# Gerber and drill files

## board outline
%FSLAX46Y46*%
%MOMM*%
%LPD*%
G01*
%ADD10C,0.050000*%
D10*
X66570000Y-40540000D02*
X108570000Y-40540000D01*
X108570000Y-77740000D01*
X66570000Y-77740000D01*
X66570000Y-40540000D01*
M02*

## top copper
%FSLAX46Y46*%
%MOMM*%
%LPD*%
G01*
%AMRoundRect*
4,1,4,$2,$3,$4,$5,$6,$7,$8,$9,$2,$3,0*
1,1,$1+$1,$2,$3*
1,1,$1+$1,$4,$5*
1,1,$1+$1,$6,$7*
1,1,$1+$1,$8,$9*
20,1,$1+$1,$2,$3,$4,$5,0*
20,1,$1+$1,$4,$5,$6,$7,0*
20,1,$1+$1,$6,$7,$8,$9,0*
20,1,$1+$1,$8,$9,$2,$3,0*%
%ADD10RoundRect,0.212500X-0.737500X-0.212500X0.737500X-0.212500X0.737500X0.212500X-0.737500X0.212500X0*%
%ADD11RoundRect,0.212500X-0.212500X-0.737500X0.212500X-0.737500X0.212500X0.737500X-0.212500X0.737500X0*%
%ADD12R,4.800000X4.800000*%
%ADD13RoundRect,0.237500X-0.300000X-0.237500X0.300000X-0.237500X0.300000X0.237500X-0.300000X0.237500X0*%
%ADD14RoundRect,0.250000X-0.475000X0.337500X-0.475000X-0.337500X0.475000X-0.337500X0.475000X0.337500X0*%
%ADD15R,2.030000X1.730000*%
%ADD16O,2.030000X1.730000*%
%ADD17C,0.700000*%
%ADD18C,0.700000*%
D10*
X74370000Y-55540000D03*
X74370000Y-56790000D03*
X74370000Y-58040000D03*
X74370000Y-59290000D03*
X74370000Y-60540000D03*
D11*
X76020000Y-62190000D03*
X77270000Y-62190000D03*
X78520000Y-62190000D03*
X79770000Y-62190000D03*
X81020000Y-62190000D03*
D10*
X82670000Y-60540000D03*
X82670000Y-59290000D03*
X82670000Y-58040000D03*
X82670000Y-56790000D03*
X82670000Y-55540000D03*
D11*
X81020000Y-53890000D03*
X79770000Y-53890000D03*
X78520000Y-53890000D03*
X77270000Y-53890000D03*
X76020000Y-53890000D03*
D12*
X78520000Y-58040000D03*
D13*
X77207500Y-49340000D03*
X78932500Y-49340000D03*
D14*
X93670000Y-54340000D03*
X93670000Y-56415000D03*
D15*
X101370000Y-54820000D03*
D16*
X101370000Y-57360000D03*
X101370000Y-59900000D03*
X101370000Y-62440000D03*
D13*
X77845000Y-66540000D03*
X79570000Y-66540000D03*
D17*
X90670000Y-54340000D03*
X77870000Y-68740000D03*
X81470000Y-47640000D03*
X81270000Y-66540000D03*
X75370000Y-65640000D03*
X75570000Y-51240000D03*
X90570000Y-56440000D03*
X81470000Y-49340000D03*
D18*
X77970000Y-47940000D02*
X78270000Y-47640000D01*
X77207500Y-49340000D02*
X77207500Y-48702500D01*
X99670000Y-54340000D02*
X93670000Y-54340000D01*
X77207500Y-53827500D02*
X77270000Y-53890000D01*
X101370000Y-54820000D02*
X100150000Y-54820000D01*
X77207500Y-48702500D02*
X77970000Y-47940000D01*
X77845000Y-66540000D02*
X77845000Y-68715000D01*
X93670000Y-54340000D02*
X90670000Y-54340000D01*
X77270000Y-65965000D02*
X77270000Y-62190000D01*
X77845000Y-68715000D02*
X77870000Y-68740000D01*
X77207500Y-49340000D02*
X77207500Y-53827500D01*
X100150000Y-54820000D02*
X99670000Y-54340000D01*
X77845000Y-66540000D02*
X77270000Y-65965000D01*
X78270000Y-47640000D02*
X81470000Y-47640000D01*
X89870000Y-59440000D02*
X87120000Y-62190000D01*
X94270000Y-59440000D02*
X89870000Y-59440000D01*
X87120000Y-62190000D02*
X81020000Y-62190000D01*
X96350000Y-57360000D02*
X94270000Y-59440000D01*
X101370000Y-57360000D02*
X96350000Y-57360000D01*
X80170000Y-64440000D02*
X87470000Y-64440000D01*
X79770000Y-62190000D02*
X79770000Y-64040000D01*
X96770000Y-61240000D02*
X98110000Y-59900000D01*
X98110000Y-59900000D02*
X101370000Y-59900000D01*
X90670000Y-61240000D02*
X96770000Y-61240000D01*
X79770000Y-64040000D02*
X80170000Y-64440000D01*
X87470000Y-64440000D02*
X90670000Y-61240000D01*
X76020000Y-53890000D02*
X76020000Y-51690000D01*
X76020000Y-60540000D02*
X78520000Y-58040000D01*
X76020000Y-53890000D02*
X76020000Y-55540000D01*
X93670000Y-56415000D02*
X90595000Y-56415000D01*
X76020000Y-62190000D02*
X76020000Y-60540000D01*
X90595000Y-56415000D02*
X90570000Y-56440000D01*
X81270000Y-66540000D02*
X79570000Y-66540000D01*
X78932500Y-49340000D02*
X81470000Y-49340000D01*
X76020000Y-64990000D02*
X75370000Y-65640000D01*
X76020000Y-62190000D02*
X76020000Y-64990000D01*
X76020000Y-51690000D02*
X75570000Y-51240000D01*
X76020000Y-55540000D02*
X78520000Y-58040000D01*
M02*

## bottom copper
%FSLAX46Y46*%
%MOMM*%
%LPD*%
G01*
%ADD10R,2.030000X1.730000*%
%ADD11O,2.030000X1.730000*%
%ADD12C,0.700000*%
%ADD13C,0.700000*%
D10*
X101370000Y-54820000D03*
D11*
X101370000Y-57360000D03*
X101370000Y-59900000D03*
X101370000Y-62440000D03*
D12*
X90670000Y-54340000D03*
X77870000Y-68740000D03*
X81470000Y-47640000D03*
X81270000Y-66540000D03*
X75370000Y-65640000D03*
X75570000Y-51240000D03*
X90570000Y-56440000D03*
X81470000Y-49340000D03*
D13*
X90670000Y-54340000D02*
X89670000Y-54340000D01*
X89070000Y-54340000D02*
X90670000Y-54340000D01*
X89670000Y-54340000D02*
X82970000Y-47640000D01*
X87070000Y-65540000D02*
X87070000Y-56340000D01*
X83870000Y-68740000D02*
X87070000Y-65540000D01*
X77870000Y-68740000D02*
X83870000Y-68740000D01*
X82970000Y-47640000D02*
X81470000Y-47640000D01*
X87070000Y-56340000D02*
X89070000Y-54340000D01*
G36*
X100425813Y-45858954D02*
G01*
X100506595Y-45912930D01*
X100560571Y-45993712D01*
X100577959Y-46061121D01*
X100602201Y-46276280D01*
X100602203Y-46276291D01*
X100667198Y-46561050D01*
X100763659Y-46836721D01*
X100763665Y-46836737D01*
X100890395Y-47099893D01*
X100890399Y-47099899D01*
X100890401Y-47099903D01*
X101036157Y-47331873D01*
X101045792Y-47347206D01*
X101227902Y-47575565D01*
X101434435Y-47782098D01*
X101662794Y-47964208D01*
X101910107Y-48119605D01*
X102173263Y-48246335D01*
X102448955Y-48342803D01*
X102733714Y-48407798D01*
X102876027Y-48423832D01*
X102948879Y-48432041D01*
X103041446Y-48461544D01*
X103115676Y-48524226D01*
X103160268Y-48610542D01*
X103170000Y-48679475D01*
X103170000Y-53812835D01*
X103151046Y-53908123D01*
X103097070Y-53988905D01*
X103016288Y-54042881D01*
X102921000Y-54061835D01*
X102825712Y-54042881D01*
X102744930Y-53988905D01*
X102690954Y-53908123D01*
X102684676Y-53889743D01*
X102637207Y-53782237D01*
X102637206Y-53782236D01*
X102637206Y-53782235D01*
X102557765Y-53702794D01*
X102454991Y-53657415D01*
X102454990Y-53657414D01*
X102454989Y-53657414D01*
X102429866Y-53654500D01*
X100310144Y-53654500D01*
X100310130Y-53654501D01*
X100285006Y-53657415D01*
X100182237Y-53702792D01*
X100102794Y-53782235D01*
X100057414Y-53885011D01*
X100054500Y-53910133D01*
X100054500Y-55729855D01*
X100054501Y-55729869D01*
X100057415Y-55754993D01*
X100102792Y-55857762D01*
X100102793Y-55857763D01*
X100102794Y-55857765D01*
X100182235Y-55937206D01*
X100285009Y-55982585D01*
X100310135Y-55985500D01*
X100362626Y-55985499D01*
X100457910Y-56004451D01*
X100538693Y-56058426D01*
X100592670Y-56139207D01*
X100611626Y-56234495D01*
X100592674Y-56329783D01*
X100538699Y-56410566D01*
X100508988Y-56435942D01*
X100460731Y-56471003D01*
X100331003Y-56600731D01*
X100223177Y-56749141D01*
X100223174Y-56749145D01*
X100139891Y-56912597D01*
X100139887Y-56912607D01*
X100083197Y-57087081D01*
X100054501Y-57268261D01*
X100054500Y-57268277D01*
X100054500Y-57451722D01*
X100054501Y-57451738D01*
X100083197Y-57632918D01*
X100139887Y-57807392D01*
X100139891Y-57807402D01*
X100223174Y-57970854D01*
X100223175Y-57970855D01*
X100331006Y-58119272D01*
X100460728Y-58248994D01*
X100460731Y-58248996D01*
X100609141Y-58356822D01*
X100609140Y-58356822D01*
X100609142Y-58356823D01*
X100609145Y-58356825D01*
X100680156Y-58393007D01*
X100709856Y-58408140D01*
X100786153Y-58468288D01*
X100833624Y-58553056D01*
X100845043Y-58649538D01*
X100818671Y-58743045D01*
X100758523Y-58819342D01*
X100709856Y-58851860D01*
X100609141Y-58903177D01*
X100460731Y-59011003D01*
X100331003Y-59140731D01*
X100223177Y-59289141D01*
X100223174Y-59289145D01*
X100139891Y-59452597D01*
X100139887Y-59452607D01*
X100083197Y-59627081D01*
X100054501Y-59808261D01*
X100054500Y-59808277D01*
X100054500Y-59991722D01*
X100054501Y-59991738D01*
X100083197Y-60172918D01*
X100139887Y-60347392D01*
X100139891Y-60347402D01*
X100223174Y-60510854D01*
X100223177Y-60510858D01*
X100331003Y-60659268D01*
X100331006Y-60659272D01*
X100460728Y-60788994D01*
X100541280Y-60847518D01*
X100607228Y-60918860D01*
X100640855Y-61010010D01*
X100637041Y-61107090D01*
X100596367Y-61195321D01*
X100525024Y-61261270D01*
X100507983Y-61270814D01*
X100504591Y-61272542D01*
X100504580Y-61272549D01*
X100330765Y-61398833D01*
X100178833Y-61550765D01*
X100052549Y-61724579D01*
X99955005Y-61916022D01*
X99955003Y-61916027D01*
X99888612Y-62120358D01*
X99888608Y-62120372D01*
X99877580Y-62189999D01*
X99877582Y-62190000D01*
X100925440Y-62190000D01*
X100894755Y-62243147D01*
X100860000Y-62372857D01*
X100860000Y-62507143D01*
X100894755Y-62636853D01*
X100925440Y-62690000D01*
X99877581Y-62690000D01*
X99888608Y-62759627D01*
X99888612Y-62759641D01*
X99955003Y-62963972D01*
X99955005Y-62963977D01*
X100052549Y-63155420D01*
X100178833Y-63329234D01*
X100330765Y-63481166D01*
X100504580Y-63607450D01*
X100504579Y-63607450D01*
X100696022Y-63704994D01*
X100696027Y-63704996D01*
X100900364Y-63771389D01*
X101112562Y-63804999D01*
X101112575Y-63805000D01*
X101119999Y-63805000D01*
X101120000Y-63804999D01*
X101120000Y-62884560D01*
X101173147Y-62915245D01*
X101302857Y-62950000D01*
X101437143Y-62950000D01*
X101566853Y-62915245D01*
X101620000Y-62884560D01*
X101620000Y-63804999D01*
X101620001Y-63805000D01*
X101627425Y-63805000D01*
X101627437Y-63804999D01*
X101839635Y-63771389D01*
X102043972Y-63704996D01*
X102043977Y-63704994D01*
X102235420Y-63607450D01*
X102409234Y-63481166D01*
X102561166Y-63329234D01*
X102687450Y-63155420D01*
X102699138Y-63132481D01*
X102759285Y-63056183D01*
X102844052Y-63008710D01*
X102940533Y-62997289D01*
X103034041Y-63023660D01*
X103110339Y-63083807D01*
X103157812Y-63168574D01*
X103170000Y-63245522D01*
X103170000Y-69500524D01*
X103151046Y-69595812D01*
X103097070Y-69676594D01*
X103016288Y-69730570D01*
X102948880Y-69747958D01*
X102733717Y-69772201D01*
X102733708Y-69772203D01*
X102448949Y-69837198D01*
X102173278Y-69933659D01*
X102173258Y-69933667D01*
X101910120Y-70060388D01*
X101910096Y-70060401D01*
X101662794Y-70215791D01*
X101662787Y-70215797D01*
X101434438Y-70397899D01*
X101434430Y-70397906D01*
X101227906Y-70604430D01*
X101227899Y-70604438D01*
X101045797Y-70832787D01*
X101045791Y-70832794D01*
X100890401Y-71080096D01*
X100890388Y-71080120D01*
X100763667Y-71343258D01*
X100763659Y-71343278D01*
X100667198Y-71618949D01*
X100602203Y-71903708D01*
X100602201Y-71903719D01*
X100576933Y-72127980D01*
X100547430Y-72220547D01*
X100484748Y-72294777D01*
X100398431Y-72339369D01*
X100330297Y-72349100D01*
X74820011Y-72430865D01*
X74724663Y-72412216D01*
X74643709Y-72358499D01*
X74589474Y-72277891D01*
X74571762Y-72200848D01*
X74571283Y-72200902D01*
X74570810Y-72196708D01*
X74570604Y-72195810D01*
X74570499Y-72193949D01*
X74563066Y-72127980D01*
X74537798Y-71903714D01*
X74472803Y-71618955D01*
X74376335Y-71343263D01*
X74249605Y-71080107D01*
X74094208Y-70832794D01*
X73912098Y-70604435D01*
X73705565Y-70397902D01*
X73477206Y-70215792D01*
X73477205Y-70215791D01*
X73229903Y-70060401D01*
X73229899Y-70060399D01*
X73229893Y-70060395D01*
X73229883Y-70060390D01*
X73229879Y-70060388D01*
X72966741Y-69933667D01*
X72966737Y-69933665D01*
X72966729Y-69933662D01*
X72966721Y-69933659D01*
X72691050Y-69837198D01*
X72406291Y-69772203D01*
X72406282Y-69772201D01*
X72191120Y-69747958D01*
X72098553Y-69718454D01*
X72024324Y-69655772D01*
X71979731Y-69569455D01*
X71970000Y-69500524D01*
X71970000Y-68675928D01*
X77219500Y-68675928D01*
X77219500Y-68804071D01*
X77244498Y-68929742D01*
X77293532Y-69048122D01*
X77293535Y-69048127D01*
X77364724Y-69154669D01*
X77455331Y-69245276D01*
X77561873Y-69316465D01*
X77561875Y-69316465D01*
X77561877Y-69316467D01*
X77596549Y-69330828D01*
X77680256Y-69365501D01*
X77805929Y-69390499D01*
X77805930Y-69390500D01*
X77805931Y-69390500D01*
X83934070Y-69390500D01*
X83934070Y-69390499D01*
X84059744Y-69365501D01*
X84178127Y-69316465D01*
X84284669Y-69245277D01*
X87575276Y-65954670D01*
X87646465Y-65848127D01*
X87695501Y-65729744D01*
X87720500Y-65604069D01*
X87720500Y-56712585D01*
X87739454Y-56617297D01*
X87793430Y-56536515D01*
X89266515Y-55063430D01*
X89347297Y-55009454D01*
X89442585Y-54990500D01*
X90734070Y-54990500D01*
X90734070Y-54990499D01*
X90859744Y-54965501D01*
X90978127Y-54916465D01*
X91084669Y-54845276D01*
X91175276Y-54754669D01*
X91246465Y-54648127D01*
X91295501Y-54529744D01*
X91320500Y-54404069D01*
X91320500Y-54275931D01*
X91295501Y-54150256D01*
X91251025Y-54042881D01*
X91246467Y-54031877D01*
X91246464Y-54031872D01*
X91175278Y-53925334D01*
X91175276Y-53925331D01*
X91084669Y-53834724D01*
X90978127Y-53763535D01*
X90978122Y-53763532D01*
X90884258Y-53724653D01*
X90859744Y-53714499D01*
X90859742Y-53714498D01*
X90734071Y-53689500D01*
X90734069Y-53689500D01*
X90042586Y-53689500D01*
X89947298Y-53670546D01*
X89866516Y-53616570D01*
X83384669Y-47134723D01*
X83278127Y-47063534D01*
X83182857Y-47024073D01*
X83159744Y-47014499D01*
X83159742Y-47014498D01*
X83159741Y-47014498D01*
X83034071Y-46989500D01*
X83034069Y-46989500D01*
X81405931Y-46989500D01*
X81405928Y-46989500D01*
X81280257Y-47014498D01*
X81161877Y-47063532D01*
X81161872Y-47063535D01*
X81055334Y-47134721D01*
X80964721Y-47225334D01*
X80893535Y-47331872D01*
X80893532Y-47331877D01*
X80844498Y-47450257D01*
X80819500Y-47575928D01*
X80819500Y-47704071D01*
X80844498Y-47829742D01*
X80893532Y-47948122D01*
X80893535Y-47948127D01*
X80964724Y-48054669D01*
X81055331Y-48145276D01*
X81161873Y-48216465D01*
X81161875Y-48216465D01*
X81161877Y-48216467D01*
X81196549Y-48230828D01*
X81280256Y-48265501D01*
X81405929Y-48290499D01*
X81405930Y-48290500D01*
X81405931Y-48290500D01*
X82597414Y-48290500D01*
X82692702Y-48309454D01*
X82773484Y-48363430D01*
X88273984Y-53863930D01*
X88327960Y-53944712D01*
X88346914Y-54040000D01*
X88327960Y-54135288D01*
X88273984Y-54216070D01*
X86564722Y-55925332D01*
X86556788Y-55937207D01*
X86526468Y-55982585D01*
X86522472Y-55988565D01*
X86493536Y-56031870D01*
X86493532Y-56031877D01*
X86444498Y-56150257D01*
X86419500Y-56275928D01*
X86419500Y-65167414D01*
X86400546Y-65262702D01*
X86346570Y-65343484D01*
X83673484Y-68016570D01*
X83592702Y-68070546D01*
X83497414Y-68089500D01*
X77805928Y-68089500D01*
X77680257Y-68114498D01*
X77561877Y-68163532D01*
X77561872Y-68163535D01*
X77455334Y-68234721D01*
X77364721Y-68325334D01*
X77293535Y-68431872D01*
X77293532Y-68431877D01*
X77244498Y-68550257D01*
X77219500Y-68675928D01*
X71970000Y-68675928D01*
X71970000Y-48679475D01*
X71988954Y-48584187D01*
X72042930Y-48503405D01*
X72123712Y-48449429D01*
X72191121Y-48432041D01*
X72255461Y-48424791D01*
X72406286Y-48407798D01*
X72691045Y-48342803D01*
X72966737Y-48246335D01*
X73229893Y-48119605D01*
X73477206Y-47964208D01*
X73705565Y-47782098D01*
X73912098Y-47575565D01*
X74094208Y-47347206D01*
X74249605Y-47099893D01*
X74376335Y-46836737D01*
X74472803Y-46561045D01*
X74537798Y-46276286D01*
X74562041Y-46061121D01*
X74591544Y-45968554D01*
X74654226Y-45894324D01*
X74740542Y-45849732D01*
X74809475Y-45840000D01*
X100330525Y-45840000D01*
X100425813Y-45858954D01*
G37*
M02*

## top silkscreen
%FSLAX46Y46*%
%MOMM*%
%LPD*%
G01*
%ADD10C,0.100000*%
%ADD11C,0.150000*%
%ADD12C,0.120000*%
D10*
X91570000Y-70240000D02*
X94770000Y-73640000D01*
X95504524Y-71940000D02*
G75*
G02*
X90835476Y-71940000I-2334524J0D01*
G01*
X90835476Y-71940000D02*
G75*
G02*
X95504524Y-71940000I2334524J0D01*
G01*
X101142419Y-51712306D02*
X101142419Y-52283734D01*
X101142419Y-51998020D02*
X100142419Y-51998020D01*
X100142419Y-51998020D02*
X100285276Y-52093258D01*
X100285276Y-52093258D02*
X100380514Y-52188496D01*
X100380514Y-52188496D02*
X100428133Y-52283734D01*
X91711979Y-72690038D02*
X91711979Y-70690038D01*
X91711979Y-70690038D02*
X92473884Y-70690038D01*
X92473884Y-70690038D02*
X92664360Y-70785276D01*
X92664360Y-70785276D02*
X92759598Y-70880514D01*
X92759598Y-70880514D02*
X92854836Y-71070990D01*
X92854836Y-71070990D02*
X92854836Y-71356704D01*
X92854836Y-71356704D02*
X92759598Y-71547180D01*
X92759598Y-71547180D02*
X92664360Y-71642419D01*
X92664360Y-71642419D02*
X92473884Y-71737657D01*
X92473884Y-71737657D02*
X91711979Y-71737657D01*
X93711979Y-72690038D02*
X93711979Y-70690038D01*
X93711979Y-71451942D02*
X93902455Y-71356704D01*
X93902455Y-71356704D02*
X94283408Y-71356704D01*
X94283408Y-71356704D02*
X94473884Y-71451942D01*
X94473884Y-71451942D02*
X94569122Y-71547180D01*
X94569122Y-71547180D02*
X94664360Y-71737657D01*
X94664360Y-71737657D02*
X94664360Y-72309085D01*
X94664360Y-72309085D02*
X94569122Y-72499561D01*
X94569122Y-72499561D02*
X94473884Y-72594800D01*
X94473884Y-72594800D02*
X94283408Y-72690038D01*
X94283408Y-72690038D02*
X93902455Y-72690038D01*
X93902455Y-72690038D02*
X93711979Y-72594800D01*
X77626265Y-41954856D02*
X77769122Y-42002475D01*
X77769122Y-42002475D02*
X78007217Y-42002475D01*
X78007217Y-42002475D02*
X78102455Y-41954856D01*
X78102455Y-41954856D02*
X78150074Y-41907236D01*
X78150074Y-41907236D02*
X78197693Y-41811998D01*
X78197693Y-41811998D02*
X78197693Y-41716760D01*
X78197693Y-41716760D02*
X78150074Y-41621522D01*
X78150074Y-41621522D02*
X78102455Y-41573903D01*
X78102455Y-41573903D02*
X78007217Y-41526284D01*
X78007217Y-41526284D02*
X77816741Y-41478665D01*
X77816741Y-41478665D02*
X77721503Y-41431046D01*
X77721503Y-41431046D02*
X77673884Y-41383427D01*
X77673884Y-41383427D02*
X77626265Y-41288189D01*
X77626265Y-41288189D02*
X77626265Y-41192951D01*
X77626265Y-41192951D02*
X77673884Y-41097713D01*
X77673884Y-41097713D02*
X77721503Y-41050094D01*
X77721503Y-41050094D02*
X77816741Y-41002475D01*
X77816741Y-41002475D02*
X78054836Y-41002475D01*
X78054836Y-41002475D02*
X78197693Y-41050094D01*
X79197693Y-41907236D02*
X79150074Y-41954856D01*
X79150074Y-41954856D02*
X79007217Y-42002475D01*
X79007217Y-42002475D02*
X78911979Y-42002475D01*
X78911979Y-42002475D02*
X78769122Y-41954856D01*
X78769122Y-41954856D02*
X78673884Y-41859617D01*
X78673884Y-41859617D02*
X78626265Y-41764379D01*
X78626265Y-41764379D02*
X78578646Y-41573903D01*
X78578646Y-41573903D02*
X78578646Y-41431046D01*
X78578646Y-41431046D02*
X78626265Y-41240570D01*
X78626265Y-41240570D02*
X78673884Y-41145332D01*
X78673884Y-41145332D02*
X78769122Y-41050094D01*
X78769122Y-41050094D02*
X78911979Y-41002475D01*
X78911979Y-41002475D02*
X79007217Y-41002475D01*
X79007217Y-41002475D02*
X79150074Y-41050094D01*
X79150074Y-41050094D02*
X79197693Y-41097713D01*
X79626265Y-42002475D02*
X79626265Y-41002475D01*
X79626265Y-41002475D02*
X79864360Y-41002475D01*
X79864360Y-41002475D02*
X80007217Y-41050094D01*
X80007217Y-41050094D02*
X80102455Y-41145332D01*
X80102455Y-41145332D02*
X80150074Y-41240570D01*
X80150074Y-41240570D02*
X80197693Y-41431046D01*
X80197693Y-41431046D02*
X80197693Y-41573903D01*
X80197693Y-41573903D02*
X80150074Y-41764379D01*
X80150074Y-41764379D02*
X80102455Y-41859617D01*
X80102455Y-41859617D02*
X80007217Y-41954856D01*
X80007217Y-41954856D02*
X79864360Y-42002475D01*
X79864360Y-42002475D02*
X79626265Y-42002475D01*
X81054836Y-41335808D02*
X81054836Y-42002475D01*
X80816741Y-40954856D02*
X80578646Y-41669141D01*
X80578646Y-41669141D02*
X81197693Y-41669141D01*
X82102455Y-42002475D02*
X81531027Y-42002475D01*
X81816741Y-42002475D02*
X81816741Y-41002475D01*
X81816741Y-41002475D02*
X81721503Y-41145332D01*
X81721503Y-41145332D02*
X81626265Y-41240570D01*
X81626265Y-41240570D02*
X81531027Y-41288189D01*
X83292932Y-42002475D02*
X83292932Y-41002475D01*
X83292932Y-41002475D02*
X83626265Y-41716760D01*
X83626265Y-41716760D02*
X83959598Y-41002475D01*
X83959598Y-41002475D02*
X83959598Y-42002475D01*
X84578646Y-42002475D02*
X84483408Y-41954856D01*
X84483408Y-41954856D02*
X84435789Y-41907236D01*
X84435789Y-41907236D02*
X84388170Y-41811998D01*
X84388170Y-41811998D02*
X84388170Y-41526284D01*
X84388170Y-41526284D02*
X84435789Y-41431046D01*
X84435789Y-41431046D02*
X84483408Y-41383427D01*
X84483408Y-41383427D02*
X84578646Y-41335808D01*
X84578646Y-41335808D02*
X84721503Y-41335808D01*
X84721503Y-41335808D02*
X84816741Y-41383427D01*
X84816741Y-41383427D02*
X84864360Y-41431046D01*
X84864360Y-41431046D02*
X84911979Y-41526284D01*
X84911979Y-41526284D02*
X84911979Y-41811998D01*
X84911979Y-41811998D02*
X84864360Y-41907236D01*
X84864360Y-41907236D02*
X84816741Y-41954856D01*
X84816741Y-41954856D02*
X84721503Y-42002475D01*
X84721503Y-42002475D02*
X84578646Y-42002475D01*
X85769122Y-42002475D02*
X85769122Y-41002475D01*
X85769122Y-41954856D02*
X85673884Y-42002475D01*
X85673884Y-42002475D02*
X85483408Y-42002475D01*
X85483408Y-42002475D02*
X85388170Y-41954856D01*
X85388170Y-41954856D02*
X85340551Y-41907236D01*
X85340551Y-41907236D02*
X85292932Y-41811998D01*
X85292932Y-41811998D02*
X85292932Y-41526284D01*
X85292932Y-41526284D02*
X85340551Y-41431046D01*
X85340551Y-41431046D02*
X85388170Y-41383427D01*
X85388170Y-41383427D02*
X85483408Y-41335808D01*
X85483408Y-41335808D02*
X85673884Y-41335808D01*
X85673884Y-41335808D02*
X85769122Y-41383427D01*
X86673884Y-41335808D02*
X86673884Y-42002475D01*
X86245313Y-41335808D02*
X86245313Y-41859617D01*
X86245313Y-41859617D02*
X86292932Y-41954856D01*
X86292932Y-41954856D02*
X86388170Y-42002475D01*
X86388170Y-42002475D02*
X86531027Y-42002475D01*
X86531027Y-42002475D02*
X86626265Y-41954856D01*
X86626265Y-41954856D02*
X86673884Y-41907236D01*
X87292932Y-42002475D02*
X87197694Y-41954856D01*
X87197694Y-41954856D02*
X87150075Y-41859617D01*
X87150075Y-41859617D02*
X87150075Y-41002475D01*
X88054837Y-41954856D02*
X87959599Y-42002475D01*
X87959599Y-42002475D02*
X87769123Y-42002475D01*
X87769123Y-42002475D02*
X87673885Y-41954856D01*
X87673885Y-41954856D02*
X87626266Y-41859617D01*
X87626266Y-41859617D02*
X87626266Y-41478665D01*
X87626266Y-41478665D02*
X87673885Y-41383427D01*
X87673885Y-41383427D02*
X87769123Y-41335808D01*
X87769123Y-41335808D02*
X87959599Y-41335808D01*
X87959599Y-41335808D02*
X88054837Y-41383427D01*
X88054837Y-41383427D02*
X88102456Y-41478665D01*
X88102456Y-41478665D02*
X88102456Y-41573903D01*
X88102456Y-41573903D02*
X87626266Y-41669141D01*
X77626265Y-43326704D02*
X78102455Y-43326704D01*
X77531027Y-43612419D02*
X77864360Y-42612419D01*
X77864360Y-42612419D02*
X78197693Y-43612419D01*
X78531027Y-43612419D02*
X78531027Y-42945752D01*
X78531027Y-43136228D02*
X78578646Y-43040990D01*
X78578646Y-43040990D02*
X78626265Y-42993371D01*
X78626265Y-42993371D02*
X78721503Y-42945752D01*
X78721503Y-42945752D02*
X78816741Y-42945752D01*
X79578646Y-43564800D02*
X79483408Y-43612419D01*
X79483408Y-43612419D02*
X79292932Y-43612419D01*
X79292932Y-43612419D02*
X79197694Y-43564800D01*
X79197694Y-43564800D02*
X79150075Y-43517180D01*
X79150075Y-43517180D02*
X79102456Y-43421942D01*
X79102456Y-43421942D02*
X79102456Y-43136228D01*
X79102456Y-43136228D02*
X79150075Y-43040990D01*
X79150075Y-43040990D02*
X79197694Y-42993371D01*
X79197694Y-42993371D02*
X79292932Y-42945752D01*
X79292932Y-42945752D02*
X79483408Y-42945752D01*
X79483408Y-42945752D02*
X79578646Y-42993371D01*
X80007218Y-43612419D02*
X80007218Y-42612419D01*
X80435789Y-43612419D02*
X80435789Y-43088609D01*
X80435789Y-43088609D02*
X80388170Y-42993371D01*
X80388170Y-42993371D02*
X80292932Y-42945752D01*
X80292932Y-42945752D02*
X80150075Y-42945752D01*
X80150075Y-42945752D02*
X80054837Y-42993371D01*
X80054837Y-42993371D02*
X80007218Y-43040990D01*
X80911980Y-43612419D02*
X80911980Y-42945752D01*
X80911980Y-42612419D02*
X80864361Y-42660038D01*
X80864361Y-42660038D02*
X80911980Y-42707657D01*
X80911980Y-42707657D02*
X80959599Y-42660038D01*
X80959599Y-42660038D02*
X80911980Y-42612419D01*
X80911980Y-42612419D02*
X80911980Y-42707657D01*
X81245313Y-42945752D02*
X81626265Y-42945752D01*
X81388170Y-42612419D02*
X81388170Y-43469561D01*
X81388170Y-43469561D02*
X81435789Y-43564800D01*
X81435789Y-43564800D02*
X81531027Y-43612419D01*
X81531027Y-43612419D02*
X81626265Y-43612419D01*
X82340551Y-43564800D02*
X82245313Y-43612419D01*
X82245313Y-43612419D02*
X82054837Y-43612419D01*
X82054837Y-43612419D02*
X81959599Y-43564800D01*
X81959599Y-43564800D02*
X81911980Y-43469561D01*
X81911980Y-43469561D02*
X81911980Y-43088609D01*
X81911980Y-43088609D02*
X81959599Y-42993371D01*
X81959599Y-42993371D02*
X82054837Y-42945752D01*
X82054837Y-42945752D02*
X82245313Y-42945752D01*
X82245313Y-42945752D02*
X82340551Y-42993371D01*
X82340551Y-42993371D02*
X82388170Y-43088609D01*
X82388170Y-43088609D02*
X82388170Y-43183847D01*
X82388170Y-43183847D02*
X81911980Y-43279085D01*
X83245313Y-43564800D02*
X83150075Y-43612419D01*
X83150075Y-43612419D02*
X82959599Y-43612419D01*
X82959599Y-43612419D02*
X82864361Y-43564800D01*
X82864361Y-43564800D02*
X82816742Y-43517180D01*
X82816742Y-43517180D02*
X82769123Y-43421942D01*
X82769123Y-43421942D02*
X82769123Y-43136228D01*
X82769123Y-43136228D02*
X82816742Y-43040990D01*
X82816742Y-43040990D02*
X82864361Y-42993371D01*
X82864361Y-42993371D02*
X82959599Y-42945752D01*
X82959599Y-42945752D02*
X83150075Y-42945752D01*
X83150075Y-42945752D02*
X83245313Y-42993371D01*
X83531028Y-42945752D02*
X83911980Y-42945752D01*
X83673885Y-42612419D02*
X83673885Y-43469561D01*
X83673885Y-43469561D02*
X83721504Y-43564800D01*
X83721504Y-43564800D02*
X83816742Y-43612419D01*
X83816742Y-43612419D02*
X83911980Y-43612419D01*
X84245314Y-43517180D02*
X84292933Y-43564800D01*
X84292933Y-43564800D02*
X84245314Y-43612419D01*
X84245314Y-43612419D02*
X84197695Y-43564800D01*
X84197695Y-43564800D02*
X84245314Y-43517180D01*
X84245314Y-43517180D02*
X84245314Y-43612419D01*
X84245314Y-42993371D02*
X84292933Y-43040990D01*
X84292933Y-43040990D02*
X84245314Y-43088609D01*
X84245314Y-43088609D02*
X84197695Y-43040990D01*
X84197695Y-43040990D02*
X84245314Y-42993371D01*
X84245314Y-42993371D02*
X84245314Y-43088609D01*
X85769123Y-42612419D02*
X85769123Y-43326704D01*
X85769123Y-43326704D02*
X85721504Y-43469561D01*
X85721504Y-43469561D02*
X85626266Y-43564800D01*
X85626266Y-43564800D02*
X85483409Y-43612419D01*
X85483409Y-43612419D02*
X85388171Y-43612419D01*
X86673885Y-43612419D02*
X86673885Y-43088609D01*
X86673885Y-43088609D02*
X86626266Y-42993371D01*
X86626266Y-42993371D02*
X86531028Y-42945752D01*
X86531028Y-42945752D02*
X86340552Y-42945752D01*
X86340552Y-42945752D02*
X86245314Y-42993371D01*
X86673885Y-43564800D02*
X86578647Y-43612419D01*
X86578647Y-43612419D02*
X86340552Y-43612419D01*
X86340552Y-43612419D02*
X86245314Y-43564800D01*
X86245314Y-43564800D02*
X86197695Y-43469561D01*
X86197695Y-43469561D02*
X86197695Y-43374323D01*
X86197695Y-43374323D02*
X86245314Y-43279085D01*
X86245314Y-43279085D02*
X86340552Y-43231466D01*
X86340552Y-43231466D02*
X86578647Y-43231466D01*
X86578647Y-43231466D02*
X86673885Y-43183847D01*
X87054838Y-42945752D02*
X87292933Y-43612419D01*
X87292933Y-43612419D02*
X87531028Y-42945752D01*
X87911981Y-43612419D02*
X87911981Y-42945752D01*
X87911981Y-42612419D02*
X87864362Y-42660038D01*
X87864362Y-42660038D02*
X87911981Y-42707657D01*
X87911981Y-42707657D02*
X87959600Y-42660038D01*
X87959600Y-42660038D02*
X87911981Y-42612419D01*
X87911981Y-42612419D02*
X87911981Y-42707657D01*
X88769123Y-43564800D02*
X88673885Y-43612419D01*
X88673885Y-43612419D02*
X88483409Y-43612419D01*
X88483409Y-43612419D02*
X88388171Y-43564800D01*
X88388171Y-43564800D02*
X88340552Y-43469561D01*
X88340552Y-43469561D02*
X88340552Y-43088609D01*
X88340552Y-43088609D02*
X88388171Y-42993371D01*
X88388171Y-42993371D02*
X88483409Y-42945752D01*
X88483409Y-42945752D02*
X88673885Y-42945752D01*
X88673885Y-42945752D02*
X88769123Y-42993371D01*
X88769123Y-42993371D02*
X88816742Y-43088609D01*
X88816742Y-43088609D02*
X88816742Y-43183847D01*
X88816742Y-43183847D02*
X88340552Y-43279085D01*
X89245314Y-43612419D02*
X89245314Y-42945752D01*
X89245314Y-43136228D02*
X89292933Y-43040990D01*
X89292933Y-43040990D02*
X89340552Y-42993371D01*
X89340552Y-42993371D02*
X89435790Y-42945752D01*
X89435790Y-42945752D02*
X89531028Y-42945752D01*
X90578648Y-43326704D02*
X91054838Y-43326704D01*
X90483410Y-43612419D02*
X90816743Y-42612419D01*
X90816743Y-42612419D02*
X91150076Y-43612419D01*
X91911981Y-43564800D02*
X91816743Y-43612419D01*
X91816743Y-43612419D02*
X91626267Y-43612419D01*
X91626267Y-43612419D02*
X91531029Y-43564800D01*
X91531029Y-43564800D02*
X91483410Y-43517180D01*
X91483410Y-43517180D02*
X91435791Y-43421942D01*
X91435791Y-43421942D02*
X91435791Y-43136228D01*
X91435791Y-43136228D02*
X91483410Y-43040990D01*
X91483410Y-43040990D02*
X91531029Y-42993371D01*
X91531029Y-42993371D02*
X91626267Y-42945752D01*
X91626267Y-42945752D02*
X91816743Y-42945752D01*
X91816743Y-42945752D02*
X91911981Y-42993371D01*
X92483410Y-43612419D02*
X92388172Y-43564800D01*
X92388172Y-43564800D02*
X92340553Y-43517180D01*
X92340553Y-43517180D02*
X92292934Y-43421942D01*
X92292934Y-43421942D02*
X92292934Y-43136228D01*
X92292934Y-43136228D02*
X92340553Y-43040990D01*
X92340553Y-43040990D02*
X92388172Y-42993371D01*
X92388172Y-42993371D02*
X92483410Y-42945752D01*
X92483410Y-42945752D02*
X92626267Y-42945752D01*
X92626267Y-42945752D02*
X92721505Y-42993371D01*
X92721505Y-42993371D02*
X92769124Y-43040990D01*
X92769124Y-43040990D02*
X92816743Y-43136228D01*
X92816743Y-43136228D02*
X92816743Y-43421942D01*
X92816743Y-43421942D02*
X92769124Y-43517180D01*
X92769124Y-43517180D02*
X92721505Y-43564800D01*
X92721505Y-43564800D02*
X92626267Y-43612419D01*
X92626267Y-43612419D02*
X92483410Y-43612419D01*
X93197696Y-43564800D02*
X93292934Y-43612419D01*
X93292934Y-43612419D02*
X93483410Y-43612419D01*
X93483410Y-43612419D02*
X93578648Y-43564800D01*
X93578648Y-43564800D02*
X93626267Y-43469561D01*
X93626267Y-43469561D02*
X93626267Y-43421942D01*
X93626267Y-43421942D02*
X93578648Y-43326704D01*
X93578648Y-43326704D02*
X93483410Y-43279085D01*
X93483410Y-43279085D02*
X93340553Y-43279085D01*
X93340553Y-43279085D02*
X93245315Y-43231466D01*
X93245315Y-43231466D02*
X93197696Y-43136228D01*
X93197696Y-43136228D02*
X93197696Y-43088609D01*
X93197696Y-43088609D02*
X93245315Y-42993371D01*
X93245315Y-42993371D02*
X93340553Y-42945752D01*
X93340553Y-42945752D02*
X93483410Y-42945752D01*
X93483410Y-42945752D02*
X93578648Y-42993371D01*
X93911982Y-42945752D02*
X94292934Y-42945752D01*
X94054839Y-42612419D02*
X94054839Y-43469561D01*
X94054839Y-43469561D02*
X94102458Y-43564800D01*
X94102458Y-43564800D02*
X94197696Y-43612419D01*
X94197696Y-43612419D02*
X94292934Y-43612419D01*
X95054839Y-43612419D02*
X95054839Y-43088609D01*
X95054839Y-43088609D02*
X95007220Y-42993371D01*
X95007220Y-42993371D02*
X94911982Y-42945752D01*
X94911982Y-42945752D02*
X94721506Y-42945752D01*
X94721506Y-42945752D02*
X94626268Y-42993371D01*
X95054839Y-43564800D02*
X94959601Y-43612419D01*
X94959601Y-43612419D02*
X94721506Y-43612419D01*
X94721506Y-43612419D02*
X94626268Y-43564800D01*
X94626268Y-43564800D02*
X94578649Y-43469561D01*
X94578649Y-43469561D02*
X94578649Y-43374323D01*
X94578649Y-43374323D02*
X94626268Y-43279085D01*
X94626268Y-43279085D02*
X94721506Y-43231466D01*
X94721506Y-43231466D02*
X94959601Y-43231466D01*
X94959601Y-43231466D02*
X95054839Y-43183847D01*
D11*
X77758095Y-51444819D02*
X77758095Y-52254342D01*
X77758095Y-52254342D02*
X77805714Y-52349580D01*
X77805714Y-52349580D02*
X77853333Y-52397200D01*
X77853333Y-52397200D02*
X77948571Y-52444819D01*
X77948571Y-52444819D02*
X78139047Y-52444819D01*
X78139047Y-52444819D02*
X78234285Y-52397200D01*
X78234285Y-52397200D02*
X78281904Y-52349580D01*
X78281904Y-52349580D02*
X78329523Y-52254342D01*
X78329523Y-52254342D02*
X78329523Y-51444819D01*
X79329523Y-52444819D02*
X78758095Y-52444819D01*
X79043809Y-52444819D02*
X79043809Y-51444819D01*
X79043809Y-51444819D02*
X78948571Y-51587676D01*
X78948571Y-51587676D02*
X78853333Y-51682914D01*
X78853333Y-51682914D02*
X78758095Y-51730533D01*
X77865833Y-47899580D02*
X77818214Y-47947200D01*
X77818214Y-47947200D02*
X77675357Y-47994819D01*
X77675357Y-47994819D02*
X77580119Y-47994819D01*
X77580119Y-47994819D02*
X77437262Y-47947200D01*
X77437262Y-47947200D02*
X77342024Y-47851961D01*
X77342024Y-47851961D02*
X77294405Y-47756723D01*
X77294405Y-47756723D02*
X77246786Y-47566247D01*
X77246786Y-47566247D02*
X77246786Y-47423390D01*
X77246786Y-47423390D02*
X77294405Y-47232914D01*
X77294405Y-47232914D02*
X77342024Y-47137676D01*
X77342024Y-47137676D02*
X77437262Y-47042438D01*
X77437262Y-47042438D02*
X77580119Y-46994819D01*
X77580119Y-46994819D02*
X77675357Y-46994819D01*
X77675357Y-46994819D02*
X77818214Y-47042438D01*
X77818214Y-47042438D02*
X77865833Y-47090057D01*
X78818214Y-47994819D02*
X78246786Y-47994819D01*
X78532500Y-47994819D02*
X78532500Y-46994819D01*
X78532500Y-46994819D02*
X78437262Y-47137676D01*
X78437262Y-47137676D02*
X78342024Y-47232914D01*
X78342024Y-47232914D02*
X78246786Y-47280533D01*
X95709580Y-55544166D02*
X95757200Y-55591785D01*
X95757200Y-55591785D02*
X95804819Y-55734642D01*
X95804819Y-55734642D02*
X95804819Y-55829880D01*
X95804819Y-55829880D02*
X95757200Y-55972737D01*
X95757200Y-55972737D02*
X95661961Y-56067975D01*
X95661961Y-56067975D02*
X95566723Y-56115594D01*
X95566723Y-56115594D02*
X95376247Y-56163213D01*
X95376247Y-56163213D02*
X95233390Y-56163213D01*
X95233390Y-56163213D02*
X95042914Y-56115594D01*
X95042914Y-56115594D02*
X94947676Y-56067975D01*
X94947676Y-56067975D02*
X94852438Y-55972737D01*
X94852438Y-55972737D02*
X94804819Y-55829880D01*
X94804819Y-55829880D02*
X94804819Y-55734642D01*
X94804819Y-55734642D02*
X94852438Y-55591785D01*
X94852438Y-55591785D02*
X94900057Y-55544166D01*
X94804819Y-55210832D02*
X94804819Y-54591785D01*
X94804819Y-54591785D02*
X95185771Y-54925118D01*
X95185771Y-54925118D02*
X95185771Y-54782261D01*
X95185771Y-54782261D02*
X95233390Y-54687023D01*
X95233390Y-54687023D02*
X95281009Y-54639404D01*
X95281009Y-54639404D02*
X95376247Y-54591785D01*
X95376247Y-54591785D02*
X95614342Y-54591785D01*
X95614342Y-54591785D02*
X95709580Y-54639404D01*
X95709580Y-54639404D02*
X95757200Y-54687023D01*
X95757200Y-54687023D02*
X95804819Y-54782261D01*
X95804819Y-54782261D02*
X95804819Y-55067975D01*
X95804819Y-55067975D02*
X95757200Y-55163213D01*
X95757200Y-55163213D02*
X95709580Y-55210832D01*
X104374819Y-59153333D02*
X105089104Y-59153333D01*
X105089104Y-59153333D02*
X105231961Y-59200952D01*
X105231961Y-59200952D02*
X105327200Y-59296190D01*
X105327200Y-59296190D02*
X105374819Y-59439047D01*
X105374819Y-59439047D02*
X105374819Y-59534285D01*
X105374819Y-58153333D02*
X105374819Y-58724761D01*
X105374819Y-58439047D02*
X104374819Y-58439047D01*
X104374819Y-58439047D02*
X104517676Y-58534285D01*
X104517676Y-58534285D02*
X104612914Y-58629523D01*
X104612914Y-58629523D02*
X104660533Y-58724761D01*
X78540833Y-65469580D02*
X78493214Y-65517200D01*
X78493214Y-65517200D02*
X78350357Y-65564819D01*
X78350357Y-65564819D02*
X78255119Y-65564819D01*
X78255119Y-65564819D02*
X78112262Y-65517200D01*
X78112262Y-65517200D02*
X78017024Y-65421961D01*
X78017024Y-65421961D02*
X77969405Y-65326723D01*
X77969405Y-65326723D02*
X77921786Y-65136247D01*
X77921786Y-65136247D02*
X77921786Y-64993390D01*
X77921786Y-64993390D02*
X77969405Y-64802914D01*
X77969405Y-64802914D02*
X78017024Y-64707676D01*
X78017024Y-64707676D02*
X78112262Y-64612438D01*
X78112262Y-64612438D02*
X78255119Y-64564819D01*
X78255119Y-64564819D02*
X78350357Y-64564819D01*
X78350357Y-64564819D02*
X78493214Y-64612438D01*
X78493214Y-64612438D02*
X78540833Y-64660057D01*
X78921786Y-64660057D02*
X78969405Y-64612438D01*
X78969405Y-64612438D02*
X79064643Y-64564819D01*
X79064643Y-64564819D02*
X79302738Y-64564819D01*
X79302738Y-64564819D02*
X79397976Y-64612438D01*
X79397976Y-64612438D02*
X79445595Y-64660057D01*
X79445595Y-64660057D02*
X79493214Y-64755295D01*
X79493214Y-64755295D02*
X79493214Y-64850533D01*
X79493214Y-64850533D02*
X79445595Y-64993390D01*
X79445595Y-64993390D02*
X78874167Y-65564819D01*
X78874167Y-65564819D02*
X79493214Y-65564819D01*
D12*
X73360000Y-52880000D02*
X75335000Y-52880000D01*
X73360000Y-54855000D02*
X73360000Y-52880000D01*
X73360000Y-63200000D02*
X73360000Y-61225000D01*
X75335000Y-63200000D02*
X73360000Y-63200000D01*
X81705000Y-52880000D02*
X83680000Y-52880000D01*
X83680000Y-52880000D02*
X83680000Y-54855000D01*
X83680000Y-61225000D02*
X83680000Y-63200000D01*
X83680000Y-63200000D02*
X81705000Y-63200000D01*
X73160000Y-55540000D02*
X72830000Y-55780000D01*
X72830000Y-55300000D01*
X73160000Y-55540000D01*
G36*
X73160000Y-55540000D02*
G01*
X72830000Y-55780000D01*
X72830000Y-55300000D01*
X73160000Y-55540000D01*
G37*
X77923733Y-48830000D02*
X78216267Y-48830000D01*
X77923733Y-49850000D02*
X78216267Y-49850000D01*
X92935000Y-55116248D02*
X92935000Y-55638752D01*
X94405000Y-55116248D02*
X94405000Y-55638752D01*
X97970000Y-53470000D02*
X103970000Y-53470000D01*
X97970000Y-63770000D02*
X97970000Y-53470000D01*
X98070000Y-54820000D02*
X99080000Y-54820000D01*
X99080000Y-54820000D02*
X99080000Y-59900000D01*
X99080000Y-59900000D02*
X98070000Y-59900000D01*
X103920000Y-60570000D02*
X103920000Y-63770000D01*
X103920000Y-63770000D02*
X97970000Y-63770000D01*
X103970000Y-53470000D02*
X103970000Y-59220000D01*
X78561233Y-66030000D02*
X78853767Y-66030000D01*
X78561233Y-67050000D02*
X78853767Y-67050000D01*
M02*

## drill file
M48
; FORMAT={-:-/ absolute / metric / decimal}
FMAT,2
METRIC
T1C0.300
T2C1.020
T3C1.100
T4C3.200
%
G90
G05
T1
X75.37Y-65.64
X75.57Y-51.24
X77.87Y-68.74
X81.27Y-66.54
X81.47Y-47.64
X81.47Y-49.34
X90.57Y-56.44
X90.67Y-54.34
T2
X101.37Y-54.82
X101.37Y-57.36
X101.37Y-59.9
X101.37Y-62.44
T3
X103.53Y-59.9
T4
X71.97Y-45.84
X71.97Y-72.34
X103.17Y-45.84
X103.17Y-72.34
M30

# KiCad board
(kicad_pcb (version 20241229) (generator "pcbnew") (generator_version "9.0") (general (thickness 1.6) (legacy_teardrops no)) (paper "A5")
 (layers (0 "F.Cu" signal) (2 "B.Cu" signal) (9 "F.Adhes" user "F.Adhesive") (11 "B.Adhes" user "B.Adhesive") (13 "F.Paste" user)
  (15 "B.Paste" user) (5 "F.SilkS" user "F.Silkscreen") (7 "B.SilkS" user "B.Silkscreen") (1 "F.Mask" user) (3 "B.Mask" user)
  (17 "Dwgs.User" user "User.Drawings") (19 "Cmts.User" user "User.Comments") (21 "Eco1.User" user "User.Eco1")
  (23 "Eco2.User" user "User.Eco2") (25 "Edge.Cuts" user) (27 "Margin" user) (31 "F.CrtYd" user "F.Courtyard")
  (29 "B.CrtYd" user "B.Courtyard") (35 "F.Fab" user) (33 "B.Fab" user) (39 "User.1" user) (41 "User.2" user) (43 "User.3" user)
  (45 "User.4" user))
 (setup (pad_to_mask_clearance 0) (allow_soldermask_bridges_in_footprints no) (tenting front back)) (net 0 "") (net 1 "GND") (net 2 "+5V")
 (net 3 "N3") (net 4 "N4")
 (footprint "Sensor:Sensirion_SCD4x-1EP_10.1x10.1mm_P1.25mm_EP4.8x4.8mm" (layer "F.Cu") (at 78.52 58.04)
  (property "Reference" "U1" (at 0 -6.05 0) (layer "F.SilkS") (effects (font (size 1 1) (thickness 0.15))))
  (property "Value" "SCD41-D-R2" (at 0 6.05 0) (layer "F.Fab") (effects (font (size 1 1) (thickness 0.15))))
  (fp_line (start -5.16 -5.16) (end -3.185 -5.16) (stroke (width 0.12) (type solid)) (layer "F.SilkS"))
  (fp_line (start -5.16 -3.185) (end -5.16 -5.16) (stroke (width 0.12) (type solid)) (layer "F.SilkS"))
  (fp_line (start -5.16 5.16) (end -5.16 3.185) (stroke (width 0.12) (type solid)) (layer "F.SilkS"))
  (fp_line (start -3.185 5.16) (end -5.16 5.16) (stroke (width 0.12) (type solid)) (layer "F.SilkS"))
  (fp_line (start 3.185 -5.16) (end 5.16 -5.16) (stroke (width 0.12) (type solid)) (layer "F.SilkS"))
  (fp_line (start 5.16 -5.16) (end 5.16 -3.185) (stroke (width 0.12) (type solid)) (layer "F.SilkS"))
  (fp_line (start 5.16 3.185) (end 5.16 5.16) (stroke (width 0.12) (type solid)) (layer "F.SilkS"))
  (fp_line (start 5.16 5.16) (end 3.185 5.16) (stroke (width 0.12) (type solid)) (layer "F.SilkS"))
  (fp_poly (pts (xy -5.36 -2.5) (xy -5.69 -2.26) (xy -5.69 -2.74)) (stroke (width 0.12) (type solid)) (fill yes) (layer "F.SilkS"))
  (pad "" smd roundrect (at -1.2 -1.2) (size 1.93 1.93) (layers "F.Paste") (roundrect_rratio 0.129534))
  (pad "" smd roundrect (at -1.2 1.2) (size 1.93 1.93) (layers "F.Paste") (roundrect_rratio 0.129534))
  (pad "" smd roundrect (at 1.2 -1.2) (size 1.93 1.93) (layers "F.Paste") (roundrect_rratio 0.129534))
  (pad "" smd roundrect (at 1.2 1.2) (size 1.93 1.93) (layers "F.Paste") (roundrect_rratio 0.129534))
  (pad "1" smd roundrect (at -4.15 -2.5) (size 1.9 0.85) (layers "F.Cu" "F.Mask" "F.Paste") (roundrect_rratio 0.25))
  (pad "2" smd roundrect (at -4.15 -1.25) (size 1.9 0.85) (layers "F.Cu" "F.Mask" "F.Paste") (roundrect_rratio 0.25))
  (pad "3" smd roundrect (at -4.15 0) (size 1.9 0.85) (layers "F.Cu" "F.Mask" "F.Paste") (roundrect_rratio 0.25))
  (pad "4" smd roundrect (at -4.15 1.25) (size 1.9 0.85) (layers "F.Cu" "F.Mask" "F.Paste") (roundrect_rratio 0.25))
  (pad "5" smd roundrect (at -4.15 2.5) (size 1.9 0.85) (layers "F.Cu" "F.Mask" "F.Paste") (roundrect_rratio 0.25))
  (pad "6" smd roundrect (at -2.5 4.15) (size 0.85 1.9) (layers "F.Cu" "F.Mask" "F.Paste") (roundrect_rratio 0.25) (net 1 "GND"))
  (pad "7" smd roundrect (at -1.25 4.15) (size 0.85 1.9) (layers "F.Cu" "F.Mask" "F.Paste") (roundrect_rratio 0.25) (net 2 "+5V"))
  (pad "8" smd roundrect (at 0 4.15) (size 0.85 1.9) (layers "F.Cu" "F.Mask" "F.Paste") (roundrect_rratio 0.25))
  (pad "9" smd roundrect (at 1.25 4.15) (size 0.85 1.9) (layers "F.Cu" "F.Mask" "F.Paste") (roundrect_rratio 0.25) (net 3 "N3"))
  (pad "10" smd roundrect (at 2.5 4.15) (size 0.85 1.9) (layers "F.Cu" "F.Mask" "F.Paste") (roundrect_rratio 0.25) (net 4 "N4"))
  (pad "11" smd roundrect (at 4.15 2.5) (size 1.9 0.85) (layers "F.Cu" "F.Mask" "F.Paste") (roundrect_rratio 0.25))
  (pad "12" smd roundrect (at 4.15 1.25) (size 1.9 0.85) (layers "F.Cu" "F.Mask" "F.Paste") (roundrect_rratio 0.25))
  (pad "13" smd roundrect (at 4.15 0) (size 1.9 0.85) (layers "F.Cu" "F.Mask" "F.Paste") (roundrect_rratio 0.25))
  (pad "14" smd roundrect (at 4.15 -1.25) (size 1.9 0.85) (layers "F.Cu" "F.Mask" "F.Paste") (roundrect_rratio 0.25))
  (pad "15" smd roundrect (at 4.15 -2.5) (size 1.9 0.85) (layers "F.Cu" "F.Mask" "F.Paste") (roundrect_rratio 0.25))
  (pad "16" smd roundrect (at 2.5 -4.15) (size 0.85 1.9) (layers "F.Cu" "F.Mask" "F.Paste") (roundrect_rratio 0.25))
  (pad "17" smd roundrect (at 1.25 -4.15) (size 0.85 1.9) (layers "F.Cu" "F.Mask" "F.Paste") (roundrect_rratio 0.25))
  (pad "18" smd roundrect (at 0 -4.15) (size 0.85 1.9) (layers "F.Cu" "F.Mask" "F.Paste") (roundrect_rratio 0.25))
  (pad "19" smd roundrect (at -1.25 -4.15) (size 0.85 1.9) (layers "F.Cu" "F.Mask" "F.Paste") (roundrect_rratio 0.25) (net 2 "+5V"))
  (pad "20" smd roundrect (at -2.5 -4.15) (size 0.85 1.9) (layers "F.Cu" "F.Mask" "F.Paste") (roundrect_rratio 0.25) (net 1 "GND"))
  (pad "21" smd rect (at 0 0) (size 4.8 4.8) (layers "F.Cu" "F.Mask") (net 1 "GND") (zone_connect 2)))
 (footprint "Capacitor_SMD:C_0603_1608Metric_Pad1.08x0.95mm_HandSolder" (layer "F.Cu") (at 78.07 49.34)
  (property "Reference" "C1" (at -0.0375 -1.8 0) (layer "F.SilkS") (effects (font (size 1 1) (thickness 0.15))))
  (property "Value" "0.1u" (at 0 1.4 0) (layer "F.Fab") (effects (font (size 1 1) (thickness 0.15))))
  (fp_line (start -0.146267 -0.51) (end 0.146267 -0.51) (stroke (width 0.12) (type solid)) (layer "F.SilkS"))
  (fp_line (start -0.146267 0.51) (end 0.146267 0.51) (stroke (width 0.12) (type solid)) (layer "F.SilkS"))
  (pad "1" smd roundrect (at -0.8625 0) (size 1.075 0.95) (layers "F.Cu" "F.Mask" "F.Paste") (roundrect_rratio 0.25) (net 2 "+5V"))
  (pad "2" smd roundrect (at 0.8625 0) (size 1.075 0.95) (layers "F.Cu" "F.Mask" "F.Paste") (roundrect_rratio 0.25) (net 1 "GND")))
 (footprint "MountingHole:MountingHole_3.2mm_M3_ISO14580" (layer "F.Cu") (at 103.17 72.34)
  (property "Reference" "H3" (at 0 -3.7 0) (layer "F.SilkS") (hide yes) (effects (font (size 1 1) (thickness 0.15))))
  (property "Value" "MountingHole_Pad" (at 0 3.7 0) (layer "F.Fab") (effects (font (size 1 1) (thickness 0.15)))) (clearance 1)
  (pad "" np_thru_hole circle (at 0 0) (size 3.2 3.2) (drill 3.2) (layers "*.Cu" "*.Mask")))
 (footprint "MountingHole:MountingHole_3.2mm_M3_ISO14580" (layer "F.Cu") (at 71.97 72.34)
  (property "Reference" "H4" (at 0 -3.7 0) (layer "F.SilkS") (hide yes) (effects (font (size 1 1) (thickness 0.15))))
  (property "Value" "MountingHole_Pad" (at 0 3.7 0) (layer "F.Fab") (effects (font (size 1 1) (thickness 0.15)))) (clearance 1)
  (pad "" np_thru_hole circle (at 0 0) (size 3.2 3.2) (drill 3.2) (layers "*.Cu" "*.Mask")))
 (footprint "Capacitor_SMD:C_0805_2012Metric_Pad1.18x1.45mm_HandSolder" (layer "F.Cu") (at 93.67 55.3775 -90)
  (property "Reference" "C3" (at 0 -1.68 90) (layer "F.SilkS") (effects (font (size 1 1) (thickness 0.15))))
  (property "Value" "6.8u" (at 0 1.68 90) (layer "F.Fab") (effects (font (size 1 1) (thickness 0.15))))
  (fp_line (start -0.261252 0.735) (end 0.261252 0.735) (stroke (width 0.12) (type solid)) (layer "F.SilkS"))
  (fp_line (start -0.261252 -0.735) (end 0.261252 -0.735) (stroke (width 0.12) (type solid)) (layer "F.SilkS"))
  (pad "1" smd roundrect (at -1.0375 0 270) (size 1.175 1.45) (layers "F.Cu" "F.Mask" "F.Paste") (roundrect_rratio 0.212766) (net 2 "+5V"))
  (pad "2" smd roundrect (at 1.0375 0 270) (size 1.175 1.45) (layers "F.Cu" "F.Mask" "F.Paste") (roundrect_rratio 0.212766) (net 1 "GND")))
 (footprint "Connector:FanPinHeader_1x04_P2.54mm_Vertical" (layer "F.Cu") (at 101.37 54.82 -90)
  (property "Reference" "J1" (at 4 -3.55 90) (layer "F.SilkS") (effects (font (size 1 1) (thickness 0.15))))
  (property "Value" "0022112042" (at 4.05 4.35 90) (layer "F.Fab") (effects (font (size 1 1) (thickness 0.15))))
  (fp_line (start -1.35 3.4) (end -1.35 -2.6) (stroke (width 0.12) (type solid)) (layer "F.SilkS"))
  (fp_line (start 8.95 3.4) (end -1.35 3.4) (stroke (width 0.12) (type solid)) (layer "F.SilkS"))
  (fp_line (start 0 3.3) (end 0 2.29) (stroke (width 0.12) (type solid)) (layer "F.SilkS"))
  (fp_line (start 0 2.29) (end 5.08 2.29) (stroke (width 0.12) (type solid)) (layer "F.SilkS"))
  (fp_line (start 5.08 2.29) (end 5.08 3.3) (stroke (width 0.12) (type solid)) (layer "F.SilkS"))
  (fp_line (start 5.75 -2.55) (end 8.95 -2.55) (stroke (width 0.12) (type solid)) (layer "F.SilkS"))
  (fp_line (start 8.95 -2.55) (end 8.95 3.4) (stroke (width 0.12) (type solid)) (layer "F.SilkS"))
  (fp_line (start -1.35 -2.6) (end 4.4 -2.6) (stroke (width 0.12) (type solid)) (layer "F.SilkS"))
  (pad "" np_thru_hole circle (at 5.08 -2.16) (size 1.1 1.1) (drill 1.1) (layers "*.Cu" "*.Mask"))
  (pad "1" thru_hole rect (at 0 0) (size 2.03 1.73) (drill 1.02) (layers "*.Cu" "*.Mask") (remove_unused_layers no) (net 2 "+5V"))
  (pad "2" thru_hole oval (at 2.54 0) (size 2.03 1.73) (drill 1.02) (layers "*.Cu" "*.Mask") (remove_unused_layers no) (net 4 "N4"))
  (pad "3" thru_hole oval (at 5.08 0) (size 2.03 1.73) (drill 1.02) (layers "*.Cu" "*.Mask") (remove_unused_layers no) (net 3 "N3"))
  (pad "4" thru_hole oval (at 7.62 0) (size 2.03 1.73) (drill 1.02) (layers "*.Cu" "*.Mask") (remove_unused_layers no) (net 1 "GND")))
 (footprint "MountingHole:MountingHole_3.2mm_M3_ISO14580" (layer "F.Cu") (at 71.97 45.84)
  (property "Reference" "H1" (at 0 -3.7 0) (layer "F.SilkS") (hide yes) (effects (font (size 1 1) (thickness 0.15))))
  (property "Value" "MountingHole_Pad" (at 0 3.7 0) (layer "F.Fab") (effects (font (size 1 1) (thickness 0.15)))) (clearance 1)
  (pad "" np_thru_hole circle (at 0 0) (size 3.2 3.2) (drill 3.2) (layers "*.Cu" "*.Mask")))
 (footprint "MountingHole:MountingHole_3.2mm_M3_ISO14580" (layer "F.Cu") (at 103.17 45.84)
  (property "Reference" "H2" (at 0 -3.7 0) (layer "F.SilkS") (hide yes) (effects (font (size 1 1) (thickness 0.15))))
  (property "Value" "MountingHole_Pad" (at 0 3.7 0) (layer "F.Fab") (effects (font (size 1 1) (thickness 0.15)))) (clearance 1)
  (pad "" np_thru_hole circle (at 0 0) (size 3.2 3.2) (drill 3.2) (layers "*.Cu" "*.Mask")))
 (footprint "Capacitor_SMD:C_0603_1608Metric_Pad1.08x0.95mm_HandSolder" (layer "F.Cu") (at 78.7075 66.54)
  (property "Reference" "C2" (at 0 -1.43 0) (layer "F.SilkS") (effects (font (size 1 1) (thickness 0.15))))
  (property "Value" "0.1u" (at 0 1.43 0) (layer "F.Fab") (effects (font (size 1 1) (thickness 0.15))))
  (fp_line (start -0.146267 -0.51) (end 0.146267 -0.51) (stroke (width 0.12) (type solid)) (layer "F.SilkS"))
  (fp_line (start -0.146267 0.51) (end 0.146267 0.51) (stroke (width 0.12) (type solid)) (layer "F.SilkS"))
  (pad "1" smd roundrect (at -0.8625 0) (size 1.075 0.95) (layers "F.Cu" "F.Mask" "F.Paste") (roundrect_rratio 0.25) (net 2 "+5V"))
  (pad "2" smd roundrect (at 0.8625 0) (size 1.075 0.95) (layers "F.Cu" "F.Mask" "F.Paste") (roundrect_rratio 0.25) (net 1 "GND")))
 (gr_line (start 91.57 70.24) (end 94.77 73.64) (stroke (width 0.1) (type default)) (layer "F.SilkS"))
 (gr_circle (center 93.17 71.94) (end 94.77 70.24) (stroke (width 0.1) (type default)) (fill no) (layer "F.SilkS"))
 (gr_rect (start 66.57 40.54) (end 108.57 77.74) (stroke (width 0.05) (type default)) (fill no) (layer "Edge.Cuts"))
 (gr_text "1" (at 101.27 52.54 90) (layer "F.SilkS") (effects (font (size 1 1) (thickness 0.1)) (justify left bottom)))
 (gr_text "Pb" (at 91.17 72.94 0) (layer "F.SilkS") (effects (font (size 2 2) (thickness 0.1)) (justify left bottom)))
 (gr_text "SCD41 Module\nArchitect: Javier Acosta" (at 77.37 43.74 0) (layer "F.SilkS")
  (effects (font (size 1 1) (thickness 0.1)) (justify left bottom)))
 (segment (start 77.97 47.94) (end 78.27 47.64) (width 0.7) (layer "F.Cu") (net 2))
 (segment (start 77.2075 49.34) (end 77.2075 48.7025) (width 0.7) (layer "F.Cu") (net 2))
 (segment (start 99.67 54.34) (end 93.67 54.34) (width 0.7) (layer "F.Cu") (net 2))
 (segment (start 77.2075 53.8275) (end 77.27 53.89) (width 0.7) (layer "F.Cu") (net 2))
 (segment (start 101.37 54.82) (end 100.15 54.82) (width 0.7) (layer "F.Cu") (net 2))
 (segment (start 77.2075 48.7025) (end 77.97 47.94) (width 0.7) (layer "F.Cu") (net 2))
 (segment (start 77.845 66.54) (end 77.845 68.715) (width 0.7) (layer "F.Cu") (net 2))
 (segment (start 93.67 54.34) (end 90.67 54.34) (width 0.7) (layer "F.Cu") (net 2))
 (segment (start 77.27 65.965) (end 77.27 62.19) (width 0.7) (layer "F.Cu") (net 2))
 (segment (start 77.845 68.715) (end 77.87 68.74) (width 0.7) (layer "F.Cu") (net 2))
 (segment (start 77.2075 49.34) (end 77.2075 53.8275) (width 0.7) (layer "F.Cu") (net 2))
 (segment (start 100.15 54.82) (end 99.67 54.34) (width 0.7) (layer "F.Cu") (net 2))
 (segment (start 77.845 66.54) (end 77.27 65.965) (width 0.7) (layer "F.Cu") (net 2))
 (segment (start 78.27 47.64) (end 81.47 47.64) (width 0.7) (layer "F.Cu") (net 2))
 (via (at 90.67 54.34) (size 0.7) (drill 0.3) (layers "F.Cu" "B.Cu") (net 2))
 (via (at 77.87 68.74) (size 0.7) (drill 0.3) (layers "F.Cu" "B.Cu") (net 2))
 (via (at 81.47 47.64) (size 0.7) (drill 0.3) (layers "F.Cu" "B.Cu") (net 2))
 (segment (start 90.67 54.34) (end 89.67 54.34) (width 0.7) (layer "B.Cu") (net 2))
 (segment (start 89.07 54.34) (end 90.67 54.34) (width 0.7) (layer "B.Cu") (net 2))
 (segment (start 89.67 54.34) (end 82.97 47.64) (width 0.7) (layer "B.Cu") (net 2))
 (segment (start 87.07 65.54) (end 87.07 56.34) (width 0.7) (layer "B.Cu") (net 2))
 (segment (start 83.87 68.74) (end 87.07 65.54) (width 0.7) (layer "B.Cu") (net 2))
 (segment (start 77.87 68.74) (end 83.87 68.74) (width 0.7) (layer "B.Cu") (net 2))
 (segment (start 82.97 47.64) (end 81.47 47.64) (width 0.7) (layer "B.Cu") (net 2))
 (segment (start 87.07 56.34) (end 89.07 54.34) (width 0.7) (layer "B.Cu") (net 2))
 (segment (start 89.87 59.44) (end 87.12 62.19) (width 0.7) (layer "F.Cu") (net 4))
 (segment (start 94.27 59.44) (end 89.87 59.44) (width 0.7) (layer "F.Cu") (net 4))
 (segment (start 87.12 62.19) (end 81.02 62.19) (width 0.7) (layer "F.Cu") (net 4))
 (segment (start 96.35 57.36) (end 94.27 59.44) (width 0.7) (layer "F.Cu") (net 4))
 (segment (start 101.37 57.36) (end 96.35 57.36) (width 0.7) (layer "F.Cu") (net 4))
 (segment (start 80.17 64.44) (end 87.47 64.44) (width 0.7) (layer "F.Cu") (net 3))
 (segment (start 79.77 62.19) (end 79.77 64.04) (width 0.7) (layer "F.Cu") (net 3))
 (segment (start 96.77 61.24) (end 98.11 59.9) (width 0.7) (layer "F.Cu") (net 3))
 (segment (start 98.11 59.9) (end 101.37 59.9) (width 0.7) (layer "F.Cu") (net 3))
 (segment (start 90.67 61.24) (end 96.77 61.24) (width 0.7) (layer "F.Cu") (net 3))
 (segment (start 79.77 64.04) (end 80.17 64.44) (width 0.7) (layer "F.Cu") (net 3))
 (segment (start 87.47 64.44) (end 90.67 61.24) (width 0.7) (layer "F.Cu") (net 3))
 (segment (start 76.02 53.89) (end 76.02 51.69) (width 0.7) (layer "F.Cu") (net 1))
 (segment (start 76.02 60.54) (end 78.52 58.04) (width 0.7) (layer "F.Cu") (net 1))
 (segment (start 76.02 53.89) (end 76.02 55.54) (width 0.7) (layer "F.Cu") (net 1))
 (segment (start 93.67 56.415) (end 90.595 56.415) (width 0.7) (layer "F.Cu") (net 1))
 (segment (start 76.02 62.19) (end 76.02 60.54) (width 0.7) (layer "F.Cu") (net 1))
 (segment (start 90.595 56.415) (end 90.57 56.44) (width 0.7) (layer "F.Cu") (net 1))
 (segment (start 81.27 66.54) (end 79.57 66.54) (width 0.7) (layer "F.Cu") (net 1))
 (segment (start 78.9325 49.34) (end 81.47 49.34) (width 0.7) (layer "F.Cu") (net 1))
 (segment (start 76.02 64.99) (end 75.37 65.64) (width 0.7) (layer "F.Cu") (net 1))
 (segment (start 76.02 62.19) (end 76.02 64.99) (width 0.7) (layer "F.Cu") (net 1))
 (segment (start 76.02 51.69) (end 75.57 51.24) (width 0.7) (layer "F.Cu") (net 1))
 (segment (start 76.02 55.54) (end 78.52 58.04) (width 0.7) (layer "F.Cu") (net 1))
 (via (at 81.27 66.54) (size 0.7) (drill 0.3) (layers "F.Cu" "B.Cu") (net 1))
 (via (at 75.37 65.64) (size 0.7) (drill 0.3) (layers "F.Cu" "B.Cu") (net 1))
 (via (at 75.57 51.24) (size 0.7) (drill 0.3) (layers "F.Cu" "B.Cu") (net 1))
 (via (at 90.57 56.44) (size 0.7) (drill 0.3) (layers "F.Cu" "B.Cu") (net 1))
 (via (at 81.47 49.34) (size 0.7) (drill 0.3) (layers "F.Cu" "B.Cu") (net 1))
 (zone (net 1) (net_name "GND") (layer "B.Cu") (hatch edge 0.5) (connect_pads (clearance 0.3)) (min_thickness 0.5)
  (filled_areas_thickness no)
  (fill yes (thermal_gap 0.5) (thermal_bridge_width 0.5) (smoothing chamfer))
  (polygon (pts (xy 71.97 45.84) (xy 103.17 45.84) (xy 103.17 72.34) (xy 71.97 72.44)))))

